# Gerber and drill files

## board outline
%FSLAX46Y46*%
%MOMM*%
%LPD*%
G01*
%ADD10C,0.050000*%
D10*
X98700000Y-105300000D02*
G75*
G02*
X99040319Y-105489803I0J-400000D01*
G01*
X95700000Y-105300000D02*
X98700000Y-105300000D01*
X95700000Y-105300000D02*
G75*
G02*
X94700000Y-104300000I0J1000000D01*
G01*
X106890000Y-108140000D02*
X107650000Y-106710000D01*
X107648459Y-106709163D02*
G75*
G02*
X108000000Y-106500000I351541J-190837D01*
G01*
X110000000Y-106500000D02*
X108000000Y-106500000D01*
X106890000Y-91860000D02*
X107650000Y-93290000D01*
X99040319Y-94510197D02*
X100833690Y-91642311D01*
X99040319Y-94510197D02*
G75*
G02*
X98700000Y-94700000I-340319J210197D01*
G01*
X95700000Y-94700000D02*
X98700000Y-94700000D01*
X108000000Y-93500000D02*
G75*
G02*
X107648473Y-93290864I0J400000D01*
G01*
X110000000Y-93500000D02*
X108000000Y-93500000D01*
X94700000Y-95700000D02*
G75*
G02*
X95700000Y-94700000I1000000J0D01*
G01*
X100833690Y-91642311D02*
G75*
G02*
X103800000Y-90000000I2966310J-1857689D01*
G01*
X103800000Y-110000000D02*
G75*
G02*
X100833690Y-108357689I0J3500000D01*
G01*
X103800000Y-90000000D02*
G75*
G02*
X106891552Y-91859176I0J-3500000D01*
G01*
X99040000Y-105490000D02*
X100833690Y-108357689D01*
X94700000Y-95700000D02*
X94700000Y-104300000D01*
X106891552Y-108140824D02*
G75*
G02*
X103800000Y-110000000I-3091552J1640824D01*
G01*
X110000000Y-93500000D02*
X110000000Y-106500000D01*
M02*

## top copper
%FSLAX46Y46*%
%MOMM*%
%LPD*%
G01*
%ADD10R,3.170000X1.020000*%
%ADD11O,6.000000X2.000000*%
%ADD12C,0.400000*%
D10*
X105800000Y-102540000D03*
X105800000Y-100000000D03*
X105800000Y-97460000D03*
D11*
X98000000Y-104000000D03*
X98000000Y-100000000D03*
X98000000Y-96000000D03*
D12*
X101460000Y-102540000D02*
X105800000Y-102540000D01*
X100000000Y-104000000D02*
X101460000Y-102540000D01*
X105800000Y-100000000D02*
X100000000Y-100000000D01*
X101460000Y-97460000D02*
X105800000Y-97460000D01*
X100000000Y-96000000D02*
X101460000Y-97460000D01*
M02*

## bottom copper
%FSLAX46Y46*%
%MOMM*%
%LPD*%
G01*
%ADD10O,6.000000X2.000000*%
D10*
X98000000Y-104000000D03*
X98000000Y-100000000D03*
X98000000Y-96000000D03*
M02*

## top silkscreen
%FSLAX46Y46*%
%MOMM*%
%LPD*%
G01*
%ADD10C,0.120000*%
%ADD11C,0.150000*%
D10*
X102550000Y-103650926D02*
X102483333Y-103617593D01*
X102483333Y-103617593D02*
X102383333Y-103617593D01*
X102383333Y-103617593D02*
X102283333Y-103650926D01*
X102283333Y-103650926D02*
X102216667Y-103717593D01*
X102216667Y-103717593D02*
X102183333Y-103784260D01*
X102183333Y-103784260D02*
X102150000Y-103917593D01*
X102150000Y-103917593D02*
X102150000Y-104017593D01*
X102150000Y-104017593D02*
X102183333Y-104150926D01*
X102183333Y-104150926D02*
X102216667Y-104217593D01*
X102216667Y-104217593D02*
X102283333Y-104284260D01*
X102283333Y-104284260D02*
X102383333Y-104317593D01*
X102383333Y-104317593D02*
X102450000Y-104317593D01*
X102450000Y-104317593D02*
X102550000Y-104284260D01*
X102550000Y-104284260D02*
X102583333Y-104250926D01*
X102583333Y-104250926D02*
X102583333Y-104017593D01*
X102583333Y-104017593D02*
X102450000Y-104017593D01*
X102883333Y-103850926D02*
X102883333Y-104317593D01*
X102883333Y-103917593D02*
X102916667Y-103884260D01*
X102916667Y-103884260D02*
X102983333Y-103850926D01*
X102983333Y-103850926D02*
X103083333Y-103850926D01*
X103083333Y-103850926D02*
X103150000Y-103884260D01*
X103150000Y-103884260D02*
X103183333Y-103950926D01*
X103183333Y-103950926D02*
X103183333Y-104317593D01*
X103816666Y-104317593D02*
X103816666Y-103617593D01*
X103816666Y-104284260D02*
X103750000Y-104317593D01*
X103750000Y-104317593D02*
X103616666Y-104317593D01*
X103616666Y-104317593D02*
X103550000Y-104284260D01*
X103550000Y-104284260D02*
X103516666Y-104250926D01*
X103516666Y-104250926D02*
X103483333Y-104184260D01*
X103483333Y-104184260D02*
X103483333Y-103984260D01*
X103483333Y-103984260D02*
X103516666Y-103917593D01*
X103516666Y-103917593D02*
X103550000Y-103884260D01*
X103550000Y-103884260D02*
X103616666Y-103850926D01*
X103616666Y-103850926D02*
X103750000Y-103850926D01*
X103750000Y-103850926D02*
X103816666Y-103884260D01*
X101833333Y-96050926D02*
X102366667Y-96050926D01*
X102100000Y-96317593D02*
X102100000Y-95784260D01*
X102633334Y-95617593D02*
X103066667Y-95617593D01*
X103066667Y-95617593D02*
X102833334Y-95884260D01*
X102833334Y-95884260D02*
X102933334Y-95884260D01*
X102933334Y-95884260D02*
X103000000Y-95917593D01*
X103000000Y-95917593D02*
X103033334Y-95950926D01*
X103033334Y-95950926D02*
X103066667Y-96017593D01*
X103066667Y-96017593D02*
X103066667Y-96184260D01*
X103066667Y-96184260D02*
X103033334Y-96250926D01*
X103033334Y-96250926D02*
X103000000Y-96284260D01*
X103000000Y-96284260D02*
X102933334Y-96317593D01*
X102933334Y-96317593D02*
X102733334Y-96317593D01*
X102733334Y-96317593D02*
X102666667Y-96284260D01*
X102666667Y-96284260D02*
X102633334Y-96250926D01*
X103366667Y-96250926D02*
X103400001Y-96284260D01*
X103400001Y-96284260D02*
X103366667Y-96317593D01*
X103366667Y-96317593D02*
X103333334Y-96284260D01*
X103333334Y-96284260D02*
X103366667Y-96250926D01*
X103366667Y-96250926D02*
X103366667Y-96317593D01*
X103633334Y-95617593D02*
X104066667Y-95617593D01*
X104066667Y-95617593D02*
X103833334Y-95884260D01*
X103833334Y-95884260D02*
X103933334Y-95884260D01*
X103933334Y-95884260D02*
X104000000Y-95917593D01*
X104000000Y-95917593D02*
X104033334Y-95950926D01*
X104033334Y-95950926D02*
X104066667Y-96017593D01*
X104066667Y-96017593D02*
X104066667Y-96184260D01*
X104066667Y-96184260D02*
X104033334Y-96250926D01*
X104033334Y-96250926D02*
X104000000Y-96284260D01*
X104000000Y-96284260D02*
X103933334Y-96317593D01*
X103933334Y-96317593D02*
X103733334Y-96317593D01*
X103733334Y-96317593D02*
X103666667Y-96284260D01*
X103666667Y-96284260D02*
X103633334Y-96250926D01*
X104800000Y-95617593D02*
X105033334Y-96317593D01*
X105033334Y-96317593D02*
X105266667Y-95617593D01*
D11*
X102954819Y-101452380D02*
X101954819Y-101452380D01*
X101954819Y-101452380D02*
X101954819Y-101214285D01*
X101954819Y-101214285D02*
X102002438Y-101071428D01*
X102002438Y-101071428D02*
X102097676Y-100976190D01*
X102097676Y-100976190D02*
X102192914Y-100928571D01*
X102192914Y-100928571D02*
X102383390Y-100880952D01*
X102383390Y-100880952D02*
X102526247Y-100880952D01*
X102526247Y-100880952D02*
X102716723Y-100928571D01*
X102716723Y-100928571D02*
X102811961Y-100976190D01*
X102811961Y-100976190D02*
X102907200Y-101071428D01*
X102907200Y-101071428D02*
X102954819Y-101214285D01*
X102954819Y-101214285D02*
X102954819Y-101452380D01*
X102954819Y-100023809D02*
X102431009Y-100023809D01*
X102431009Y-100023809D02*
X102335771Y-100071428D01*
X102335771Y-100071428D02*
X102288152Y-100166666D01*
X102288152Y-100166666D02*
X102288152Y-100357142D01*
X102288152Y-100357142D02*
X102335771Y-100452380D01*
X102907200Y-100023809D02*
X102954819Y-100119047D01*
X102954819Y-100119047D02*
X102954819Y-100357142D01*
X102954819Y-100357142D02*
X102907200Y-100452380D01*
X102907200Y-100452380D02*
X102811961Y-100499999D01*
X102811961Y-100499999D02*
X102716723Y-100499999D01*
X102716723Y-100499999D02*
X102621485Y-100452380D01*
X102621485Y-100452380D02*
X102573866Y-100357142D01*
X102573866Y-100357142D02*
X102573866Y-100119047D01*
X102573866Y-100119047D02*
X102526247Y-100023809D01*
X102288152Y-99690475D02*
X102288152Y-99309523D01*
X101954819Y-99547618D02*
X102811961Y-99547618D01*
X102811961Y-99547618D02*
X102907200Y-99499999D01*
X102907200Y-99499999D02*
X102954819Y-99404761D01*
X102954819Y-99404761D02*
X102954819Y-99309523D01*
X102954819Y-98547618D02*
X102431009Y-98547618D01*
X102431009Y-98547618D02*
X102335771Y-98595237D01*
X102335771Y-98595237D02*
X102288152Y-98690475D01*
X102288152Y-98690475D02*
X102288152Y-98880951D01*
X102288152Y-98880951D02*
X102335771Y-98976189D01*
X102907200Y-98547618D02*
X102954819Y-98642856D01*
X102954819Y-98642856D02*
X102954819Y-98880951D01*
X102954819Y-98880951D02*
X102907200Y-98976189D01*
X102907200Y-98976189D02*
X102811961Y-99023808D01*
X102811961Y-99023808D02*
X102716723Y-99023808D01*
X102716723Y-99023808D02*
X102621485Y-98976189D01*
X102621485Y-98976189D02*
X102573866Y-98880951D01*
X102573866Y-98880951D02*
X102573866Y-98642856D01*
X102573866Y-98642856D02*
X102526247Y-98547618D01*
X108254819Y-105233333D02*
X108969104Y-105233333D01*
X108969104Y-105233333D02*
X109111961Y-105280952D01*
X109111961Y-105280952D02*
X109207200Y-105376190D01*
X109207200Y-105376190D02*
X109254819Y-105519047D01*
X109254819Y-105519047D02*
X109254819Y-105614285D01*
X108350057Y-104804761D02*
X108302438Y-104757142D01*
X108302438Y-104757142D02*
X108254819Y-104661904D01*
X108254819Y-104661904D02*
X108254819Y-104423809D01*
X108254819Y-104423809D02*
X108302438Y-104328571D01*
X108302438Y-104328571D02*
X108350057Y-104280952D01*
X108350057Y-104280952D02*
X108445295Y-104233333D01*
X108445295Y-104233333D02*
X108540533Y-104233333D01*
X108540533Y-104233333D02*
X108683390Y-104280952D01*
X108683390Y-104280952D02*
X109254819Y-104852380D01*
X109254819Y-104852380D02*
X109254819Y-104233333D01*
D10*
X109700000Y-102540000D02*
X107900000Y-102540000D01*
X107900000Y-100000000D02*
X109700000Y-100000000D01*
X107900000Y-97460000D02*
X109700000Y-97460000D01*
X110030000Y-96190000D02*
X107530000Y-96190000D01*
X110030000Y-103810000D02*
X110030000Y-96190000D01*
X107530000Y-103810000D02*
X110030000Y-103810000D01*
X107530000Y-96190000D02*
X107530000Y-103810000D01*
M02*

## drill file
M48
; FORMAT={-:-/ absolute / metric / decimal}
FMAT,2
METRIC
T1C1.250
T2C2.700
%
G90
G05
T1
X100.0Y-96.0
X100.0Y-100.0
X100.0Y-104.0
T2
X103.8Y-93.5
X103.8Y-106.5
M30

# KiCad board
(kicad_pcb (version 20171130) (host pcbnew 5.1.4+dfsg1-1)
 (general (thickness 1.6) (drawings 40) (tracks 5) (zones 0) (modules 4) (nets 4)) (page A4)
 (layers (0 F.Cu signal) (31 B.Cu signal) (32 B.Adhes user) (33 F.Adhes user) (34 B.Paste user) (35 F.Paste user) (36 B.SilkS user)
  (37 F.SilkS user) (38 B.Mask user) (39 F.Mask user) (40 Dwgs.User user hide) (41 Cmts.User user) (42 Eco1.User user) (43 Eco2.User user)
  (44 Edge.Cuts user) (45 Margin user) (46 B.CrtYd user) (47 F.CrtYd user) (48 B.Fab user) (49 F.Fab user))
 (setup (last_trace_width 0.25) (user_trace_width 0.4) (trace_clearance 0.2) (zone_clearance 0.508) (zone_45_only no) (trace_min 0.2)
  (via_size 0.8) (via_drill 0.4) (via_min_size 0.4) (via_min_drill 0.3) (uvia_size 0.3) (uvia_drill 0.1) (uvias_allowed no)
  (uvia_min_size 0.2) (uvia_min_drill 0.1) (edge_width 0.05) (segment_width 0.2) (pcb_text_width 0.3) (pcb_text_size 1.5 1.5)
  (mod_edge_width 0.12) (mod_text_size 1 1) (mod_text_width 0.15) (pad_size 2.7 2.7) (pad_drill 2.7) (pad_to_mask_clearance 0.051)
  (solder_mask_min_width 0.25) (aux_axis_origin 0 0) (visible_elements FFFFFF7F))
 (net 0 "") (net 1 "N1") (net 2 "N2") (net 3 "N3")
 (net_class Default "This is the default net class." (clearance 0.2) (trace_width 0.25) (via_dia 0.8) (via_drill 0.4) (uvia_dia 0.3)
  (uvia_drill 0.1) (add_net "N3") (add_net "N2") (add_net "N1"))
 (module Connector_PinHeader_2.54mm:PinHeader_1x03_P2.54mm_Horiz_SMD (layer F.Cu) (at 105.8 100)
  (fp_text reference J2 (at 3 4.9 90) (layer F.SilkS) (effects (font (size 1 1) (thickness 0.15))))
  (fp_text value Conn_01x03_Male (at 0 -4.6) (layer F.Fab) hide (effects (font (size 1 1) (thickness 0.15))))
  (fp_line (start 3.9 2.54) (end 2.1 2.54) (layer F.SilkS) (width 0.12))
  (fp_line (start 2.1 0) (end 3.9 0) (layer F.SilkS) (width 0.12))
  (fp_line (start 2.1 -2.54) (end 3.9 -2.54) (layer F.SilkS) (width 0.12))
  (fp_line (start 4.23 -3.81) (end 1.73 -3.81) (layer F.SilkS) (width 0.12))
  (fp_line (start 4.23 3.81) (end 4.23 -3.81) (layer F.SilkS) (width 0.12))
  (fp_line (start 1.73 3.81) (end 4.23 3.81) (layer F.SilkS) (width 0.12))
  (fp_line (start 1.73 -3.81) (end 1.73 3.81) (layer F.SilkS) (width 0.12))
  (pad 3 smd rect (at 0 2.54) (size 3.17 1.02) (layers F.Cu F.Paste F.Mask) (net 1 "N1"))
  (pad 2 smd rect (at 0 0) (size 3.17 1.02) (layers F.Cu F.Paste F.Mask) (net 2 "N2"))
  (pad 1 smd rect (at 0 -2.54) (size 3.17 1.02) (layers F.Cu F.Paste F.Mask) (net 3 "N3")))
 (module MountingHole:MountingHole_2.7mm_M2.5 (layer F.Cu) (at 103.8 106.5)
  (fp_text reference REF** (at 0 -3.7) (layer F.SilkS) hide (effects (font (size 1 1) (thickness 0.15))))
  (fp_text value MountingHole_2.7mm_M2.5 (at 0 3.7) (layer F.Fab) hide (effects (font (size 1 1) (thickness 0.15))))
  (pad 1 np_thru_hole circle (at 0 0) (size 2.7 2.7) (drill 2.7) (layers *.Cu *.Mask)))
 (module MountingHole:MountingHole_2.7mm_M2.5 (layer F.Cu) (at 103.8 93.5)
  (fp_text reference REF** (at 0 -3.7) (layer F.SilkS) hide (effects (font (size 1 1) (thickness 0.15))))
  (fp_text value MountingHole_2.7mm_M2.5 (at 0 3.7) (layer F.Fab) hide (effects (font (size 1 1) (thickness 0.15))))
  (pad 1 np_thru_hole circle (at 0 0) (size 2.7 2.7) (drill 2.7) (layers *.Cu *.Mask)))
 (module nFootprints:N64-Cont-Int (layer F.Cu) (at 100 100)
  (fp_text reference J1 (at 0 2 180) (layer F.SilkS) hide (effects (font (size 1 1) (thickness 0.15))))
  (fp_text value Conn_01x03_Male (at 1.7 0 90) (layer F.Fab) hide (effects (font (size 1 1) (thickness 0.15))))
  (pad 3 thru_hole oval (at 0 4) (size 6 2) (drill 1.25 (offset -2 0)) (layers *.Cu *.Mask) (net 1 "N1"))
  (pad 2 thru_hole oval (at 0 0) (size 6 2) (drill 1.25 (offset -2 0)) (layers *.Cu *.Mask) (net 2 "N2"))
  (pad 1 thru_hole oval (at 0 -4) (size 6 2) (drill 1.25 (offset -2 0)) (layers *.Cu *.Mask) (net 3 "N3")))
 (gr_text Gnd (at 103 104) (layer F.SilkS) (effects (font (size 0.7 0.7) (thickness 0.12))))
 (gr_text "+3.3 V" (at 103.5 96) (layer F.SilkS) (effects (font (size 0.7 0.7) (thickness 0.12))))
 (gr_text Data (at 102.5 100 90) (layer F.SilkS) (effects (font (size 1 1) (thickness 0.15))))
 (gr_arc (start 98.7 105.7) (end 98.7 105.3) (angle 58.29857033) (layer Edge.Cuts) (width 0.05))
 (gr_line (start 95.7 105.3) (end 98.7 105.3) (layer Edge.Cuts) (width 0.05))
 (gr_arc (start 95.7 104.3) (end 94.7 104.3) (angle -90) (layer Edge.Cuts) (width 0.05))
 (gr_line (start 106.89 108.14) (end 107.65 106.71) (layer Edge.Cuts) (width 0.05))
 (gr_arc (start 108 106.9) (end 108 106.5) (angle -61.50436138) (layer Edge.Cuts) (width 0.05))
 (gr_line (start 110 106.5) (end 108 106.5) (layer Edge.Cuts) (width 0.05))
 (gr_line (start 106.89 91.86) (end 107.65 93.29) (layer Edge.Cuts) (width 0.05))
 (gr_line (start 99.040319 94.510197) (end 100.83369 91.642311) (layer Edge.Cuts) (width 0.05))
 (gr_arc (start 98.7 94.3) (end 98.7 94.7) (angle -58.29857033) (layer Edge.Cuts) (width 0.05))
 (gr_line (start 95.7 94.7) (end 98.7 94.7) (layer Edge.Cuts) (width 0.05))
 (gr_arc (start 108 93.1) (end 108 93.5) (angle 61.5) (layer Edge.Cuts) (width 0.05))
 (gr_line (start 110 93.5) (end 108 93.5) (layer Edge.Cuts) (width 0.05))
 (gr_arc (start 95.7 95.7) (end 94.7 95.7) (angle 90) (layer Edge.Cuts) (width 0.05))
 (gr_arc (start 103.8 93.5) (end 103.8 90) (angle -57.94262427) (layer Edge.Cuts) (width 0.05))
 (gr_arc (start 103.8 106.5) (end 103.8 110) (angle 57.94262427) (layer Edge.Cuts) (width 0.05))
 (gr_arc (start 103.8 93.5) (end 103.8 90) (angle 62.04312571) (layer Edge.Cuts) (width 0.05))
 (gr_line (start 99.04 105.49) (end 100.83369 108.357689) (layer Edge.Cuts) (width 0.05))
 (gr_line (start 94.7 95.7) (end 94.7 104.3) (layer Edge.Cuts) (width 0.05))
 (gr_arc (start 103.8 106.5) (end 103.8 110) (angle -62.04312571) (layer Edge.Cuts) (width 0.05))
 (gr_line (start 110 93.5) (end 110 106.5) (layer Edge.Cuts) (width 0.05))
 (segment (start 101.46 102.54) (end 105.8 102.54) (width 0.4) (layer F.Cu) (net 1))
 (segment (start 100 104) (end 101.46 102.54) (width 0.4) (layer F.Cu) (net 1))
 (segment (start 105.8 100) (end 100 100) (width 0.4) (layer F.Cu) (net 2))
 (segment (start 101.46 97.46) (end 105.8 97.46) (width 0.4) (layer F.Cu) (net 3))
 (segment (start 100 96) (end 101.46 97.46) (width 0.4) (layer F.Cu) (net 3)))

